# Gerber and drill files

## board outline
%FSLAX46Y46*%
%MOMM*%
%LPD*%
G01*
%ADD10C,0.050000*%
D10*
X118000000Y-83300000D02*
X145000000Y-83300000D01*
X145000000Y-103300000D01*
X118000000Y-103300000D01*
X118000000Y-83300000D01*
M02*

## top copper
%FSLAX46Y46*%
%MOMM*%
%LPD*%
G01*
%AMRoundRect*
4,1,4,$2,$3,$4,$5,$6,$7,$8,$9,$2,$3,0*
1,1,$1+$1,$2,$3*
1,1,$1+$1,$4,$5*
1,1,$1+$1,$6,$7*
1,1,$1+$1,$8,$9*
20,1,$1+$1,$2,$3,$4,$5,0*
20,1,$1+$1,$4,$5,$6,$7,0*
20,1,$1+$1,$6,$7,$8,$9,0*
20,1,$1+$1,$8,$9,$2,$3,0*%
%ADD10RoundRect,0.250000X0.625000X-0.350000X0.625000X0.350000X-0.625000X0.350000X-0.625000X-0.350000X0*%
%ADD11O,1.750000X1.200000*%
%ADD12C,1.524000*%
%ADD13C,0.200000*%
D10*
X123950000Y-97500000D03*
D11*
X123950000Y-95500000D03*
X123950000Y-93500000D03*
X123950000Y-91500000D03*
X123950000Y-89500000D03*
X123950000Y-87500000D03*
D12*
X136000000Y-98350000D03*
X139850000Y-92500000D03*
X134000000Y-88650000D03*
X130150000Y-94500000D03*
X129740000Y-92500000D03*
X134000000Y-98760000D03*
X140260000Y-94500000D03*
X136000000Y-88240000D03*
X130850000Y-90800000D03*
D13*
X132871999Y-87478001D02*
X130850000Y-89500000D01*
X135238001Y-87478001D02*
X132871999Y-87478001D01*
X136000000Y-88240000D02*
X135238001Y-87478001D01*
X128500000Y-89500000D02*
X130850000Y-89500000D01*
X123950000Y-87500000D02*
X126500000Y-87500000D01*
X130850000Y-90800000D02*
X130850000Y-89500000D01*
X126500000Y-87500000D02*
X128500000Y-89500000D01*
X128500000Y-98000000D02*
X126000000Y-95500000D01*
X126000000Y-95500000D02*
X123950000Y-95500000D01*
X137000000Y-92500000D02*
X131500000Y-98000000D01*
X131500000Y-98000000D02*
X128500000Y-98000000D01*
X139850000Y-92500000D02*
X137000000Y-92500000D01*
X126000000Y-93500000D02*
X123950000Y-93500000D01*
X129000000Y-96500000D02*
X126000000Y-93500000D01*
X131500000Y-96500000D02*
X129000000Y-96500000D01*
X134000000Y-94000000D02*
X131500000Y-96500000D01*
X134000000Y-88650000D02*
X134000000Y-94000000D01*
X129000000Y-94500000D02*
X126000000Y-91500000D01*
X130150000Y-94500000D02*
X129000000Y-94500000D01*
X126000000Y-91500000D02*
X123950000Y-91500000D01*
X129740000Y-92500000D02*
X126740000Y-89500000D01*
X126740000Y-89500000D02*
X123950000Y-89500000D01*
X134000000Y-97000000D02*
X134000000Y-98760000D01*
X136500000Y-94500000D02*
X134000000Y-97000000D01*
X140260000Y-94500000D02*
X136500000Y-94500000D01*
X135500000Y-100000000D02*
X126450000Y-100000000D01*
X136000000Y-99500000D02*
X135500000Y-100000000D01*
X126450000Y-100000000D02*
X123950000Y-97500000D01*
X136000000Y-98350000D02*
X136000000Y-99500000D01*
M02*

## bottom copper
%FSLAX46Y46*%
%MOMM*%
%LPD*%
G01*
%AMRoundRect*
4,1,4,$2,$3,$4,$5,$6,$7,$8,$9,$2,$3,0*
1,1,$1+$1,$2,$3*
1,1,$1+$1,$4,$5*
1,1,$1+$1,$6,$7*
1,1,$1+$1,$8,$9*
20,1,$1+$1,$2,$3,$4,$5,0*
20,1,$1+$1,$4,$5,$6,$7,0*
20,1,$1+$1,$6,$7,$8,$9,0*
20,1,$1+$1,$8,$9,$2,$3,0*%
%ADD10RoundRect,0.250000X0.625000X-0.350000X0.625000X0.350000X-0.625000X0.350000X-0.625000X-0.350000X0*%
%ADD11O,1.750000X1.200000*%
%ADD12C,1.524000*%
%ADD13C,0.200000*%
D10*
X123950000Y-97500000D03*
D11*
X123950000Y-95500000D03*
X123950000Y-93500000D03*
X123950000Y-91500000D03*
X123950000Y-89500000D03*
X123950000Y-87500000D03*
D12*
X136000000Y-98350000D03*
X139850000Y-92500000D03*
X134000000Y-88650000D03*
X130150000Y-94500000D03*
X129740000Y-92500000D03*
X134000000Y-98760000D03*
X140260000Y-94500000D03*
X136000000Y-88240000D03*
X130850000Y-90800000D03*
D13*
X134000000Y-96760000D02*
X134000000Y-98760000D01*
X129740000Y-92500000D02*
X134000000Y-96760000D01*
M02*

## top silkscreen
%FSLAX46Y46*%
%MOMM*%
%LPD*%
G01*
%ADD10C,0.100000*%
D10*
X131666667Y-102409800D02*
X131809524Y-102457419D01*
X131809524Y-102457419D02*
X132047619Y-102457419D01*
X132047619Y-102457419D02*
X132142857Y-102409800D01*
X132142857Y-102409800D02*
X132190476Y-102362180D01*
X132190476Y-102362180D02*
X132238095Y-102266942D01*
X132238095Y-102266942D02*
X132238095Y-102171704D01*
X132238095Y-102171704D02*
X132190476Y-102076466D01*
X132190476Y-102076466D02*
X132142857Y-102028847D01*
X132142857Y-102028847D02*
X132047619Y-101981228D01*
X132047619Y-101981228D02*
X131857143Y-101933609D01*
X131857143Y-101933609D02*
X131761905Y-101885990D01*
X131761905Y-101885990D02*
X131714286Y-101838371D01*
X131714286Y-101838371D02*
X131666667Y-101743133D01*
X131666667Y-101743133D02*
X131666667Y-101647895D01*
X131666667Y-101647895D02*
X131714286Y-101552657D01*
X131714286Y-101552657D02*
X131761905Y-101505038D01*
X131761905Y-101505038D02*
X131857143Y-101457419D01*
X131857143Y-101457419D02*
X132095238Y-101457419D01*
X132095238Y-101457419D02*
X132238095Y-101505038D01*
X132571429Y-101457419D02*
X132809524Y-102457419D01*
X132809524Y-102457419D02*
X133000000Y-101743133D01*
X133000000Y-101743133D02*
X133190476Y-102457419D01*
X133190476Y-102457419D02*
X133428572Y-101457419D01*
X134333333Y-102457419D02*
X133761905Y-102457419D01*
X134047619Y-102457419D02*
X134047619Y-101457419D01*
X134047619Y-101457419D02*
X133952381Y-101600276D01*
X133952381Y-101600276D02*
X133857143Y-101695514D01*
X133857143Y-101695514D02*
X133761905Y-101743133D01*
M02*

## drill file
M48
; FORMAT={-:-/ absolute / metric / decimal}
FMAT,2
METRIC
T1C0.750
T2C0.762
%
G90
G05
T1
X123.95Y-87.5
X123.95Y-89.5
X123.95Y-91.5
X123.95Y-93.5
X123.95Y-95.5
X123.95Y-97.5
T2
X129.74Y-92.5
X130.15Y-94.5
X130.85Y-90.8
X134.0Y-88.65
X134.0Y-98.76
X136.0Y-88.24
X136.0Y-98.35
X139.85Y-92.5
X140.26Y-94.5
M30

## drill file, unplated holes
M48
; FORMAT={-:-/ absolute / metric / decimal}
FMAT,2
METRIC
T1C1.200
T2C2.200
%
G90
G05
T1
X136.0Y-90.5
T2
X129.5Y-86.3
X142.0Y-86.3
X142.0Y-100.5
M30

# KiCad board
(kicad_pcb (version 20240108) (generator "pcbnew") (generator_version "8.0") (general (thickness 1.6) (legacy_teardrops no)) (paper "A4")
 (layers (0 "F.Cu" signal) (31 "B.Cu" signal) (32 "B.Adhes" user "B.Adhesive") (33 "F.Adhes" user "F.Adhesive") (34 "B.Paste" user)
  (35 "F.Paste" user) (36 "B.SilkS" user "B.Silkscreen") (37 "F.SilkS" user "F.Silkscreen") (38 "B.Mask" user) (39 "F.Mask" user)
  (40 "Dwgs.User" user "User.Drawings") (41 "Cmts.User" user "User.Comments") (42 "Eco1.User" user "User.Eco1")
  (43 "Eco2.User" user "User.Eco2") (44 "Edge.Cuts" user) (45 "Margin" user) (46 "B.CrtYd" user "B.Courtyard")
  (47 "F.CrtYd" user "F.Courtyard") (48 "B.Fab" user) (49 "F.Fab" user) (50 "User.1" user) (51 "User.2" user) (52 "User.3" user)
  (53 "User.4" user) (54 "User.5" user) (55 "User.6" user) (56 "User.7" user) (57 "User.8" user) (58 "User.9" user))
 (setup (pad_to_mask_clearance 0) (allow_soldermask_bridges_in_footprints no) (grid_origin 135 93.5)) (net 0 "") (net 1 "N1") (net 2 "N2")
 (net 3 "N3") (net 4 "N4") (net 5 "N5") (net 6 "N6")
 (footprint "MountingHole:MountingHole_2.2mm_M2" (layer "F.Cu") (at 129.5 86.3)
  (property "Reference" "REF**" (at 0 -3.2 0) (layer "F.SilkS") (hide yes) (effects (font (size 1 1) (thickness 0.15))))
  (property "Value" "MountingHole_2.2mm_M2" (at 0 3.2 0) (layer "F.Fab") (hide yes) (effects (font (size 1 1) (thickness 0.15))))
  (pad "" np_thru_hole circle (at 0 0) (size 2.2 2.2) (drill 2.2) (layers "F&B.Cu" "*.Mask")))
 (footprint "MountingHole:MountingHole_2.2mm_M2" (layer "F.Cu") (at 142 100.5)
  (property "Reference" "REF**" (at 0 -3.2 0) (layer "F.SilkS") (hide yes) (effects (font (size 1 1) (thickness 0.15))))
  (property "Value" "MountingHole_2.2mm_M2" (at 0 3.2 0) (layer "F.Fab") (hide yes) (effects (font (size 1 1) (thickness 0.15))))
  (pad "" np_thru_hole circle (at 0 0) (size 2.2 2.2) (drill 2.2) (layers "F&B.Cu" "*.Mask")))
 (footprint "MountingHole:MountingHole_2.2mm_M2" (layer "F.Cu") (at 142 86.3)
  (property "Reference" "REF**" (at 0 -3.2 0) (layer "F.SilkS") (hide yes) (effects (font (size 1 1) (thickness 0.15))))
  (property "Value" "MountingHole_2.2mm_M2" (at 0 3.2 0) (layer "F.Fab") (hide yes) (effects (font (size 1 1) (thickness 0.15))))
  (pad "" np_thru_hole circle (at 0 0) (size 2.2 2.2) (drill 2.2) (layers "F&B.Cu" "*.Mask")))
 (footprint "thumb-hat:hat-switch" (layer "F.Cu") (at 135 93.5)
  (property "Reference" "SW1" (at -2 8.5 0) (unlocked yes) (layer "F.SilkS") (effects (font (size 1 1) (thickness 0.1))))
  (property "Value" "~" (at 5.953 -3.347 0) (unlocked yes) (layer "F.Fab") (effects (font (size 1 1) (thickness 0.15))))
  (pad "" np_thru_hole circle (at 1 -3) (size 1.2 1.2) (drill 1.2) (layers "*.Mask"))
  (pad "1" thru_hole circle (at 1 4.85) (size 1.524 1.524) (drill 0.762) (layers "*.Cu" "*.Mask") (remove_unused_layers no) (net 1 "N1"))
  (pad "2" thru_hole circle (at 4.85 -1) (size 1.524 1.524) (drill 0.762) (layers "*.Cu" "*.Mask") (remove_unused_layers no) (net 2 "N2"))
  (pad "3" thru_hole circle (at -1 -4.85) (size 1.524 1.524) (drill 0.762) (layers "*.Cu" "*.Mask") (remove_unused_layers no) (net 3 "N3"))
  (pad "4" thru_hole circle (at -4.85 1) (size 1.524 1.524) (drill 0.762) (layers "*.Cu" "*.Mask") (remove_unused_layers no) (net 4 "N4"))
  (pad "5" thru_hole circle (at -5.26 -1) (size 1.524 1.524) (drill 0.762) (layers "*.Cu" "*.Mask") (remove_unused_layers no) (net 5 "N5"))
  (pad "5" thru_hole circle (at -1 5.26) (size 1.524 1.524) (drill 0.762) (layers "*.Cu" "*.Mask") (remove_unused_layers no) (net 5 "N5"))
  (pad "5" thru_hole circle (at 5.26 1) (size 1.524 1.524) (drill 0.762) (layers "*.Cu" "*.Mask") (remove_unused_layers no) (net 5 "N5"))
  (pad "6" thru_hole circle (at 1 -5.26) (size 1.524 1.524) (drill 0.762) (layers "*.Cu" "*.Mask") (remove_unused_layers no) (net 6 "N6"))
  (pad "7" thru_hole circle (at -4.15 -2.7) (size 1.524 1.524) (drill 0.762) (layers "*.Cu" "*.Mask") (remove_unused_layers no) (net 6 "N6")))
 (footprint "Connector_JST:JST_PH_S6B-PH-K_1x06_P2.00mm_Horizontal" (layer "B.Cu") (at 123.95 97.5 90)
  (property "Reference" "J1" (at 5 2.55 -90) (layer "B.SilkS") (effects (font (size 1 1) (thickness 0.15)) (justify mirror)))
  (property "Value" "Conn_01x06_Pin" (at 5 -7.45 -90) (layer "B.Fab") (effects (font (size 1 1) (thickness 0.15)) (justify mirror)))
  (pad "1" thru_hole roundrect (at 0 0 90) (size 1.2 1.75) (drill 0.75) (layers "*.Cu" "*.Mask") (remove_unused_layers no)
   (roundrect_rratio 0.208333) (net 1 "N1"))
  (pad "2" thru_hole oval (at 2 0 90) (size 1.2 1.75) (drill 0.75) (layers "*.Cu" "*.Mask") (remove_unused_layers no) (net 2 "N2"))
  (pad "3" thru_hole oval (at 4 0 90) (size 1.2 1.75) (drill 0.75) (layers "*.Cu" "*.Mask") (remove_unused_layers no) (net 3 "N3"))
  (pad "4" thru_hole oval (at 6 0 90) (size 1.2 1.75) (drill 0.75) (layers "*.Cu" "*.Mask") (remove_unused_layers no) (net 4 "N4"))
  (pad "5" thru_hole oval (at 8 0 90) (size 1.2 1.75) (drill 0.75) (layers "*.Cu" "*.Mask") (remove_unused_layers no) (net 5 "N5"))
  (pad "6" thru_hole oval (at 10 0 90) (size 1.2 1.75) (drill 0.75) (layers "*.Cu" "*.Mask") (remove_unused_layers no) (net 6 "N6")))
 (gr_rect (start 118 83.3) (end 145 103.3) (stroke (width 0.05) (type default)) (fill none) (layer "Edge.Cuts"))
 (segment (start 132.871999 87.478001) (end 130.85 89.5) (width 0.2) (layer "F.Cu") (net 6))
 (segment (start 130.85 90.8) (end 130.85 89.5) (width 0.2) (layer "F.Cu") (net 6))
 (segment (start 136 88.24) (end 135.238001 87.478001) (width 0.2) (layer "F.Cu") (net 6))
 (segment (start 135.238001 87.478001) (end 132.871999 87.478001) (width 0.2) (layer "F.Cu") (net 6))
 (segment (start 123.95 87.5) (end 126.5 87.5) (width 0.2) (layer "F.Cu") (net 6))
 (segment (start 128.5 89.5) (end 130.85 89.5) (width 0.2) (layer "F.Cu") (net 6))
 (segment (start 126.5 87.5) (end 128.5 89.5) (width 0.2) (layer "F.Cu") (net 6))
 (segment (start 136 99.5) (end 135.5 100) (width 0.2) (layer "F.Cu") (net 1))
 (segment (start 136 98.35) (end 136 99.5) (width 0.2) (layer "F.Cu") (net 1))
 (segment (start 135.5 100) (end 126.45 100) (width 0.2) (layer "F.Cu") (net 1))
 (segment (start 126.45 100) (end 123.95 97.5) (width 0.2) (layer "F.Cu") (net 1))
 (segment (start 140.26 94.5) (end 136.5 94.5) (width 0.2) (layer "F.Cu") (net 5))
 (segment (start 129.74 92.5) (end 126.74 89.5) (width 0.2) (layer "F.Cu") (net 5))
 (segment (start 126.74 89.5) (end 123.95 89.5) (width 0.2) (layer "F.Cu") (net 5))
 (segment (start 136.5 94.5) (end 134 97) (width 0.2) (layer "F.Cu") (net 5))
 (segment (start 134 97) (end 134 98.76) (width 0.2) (layer "F.Cu") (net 5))
 (segment (start 129.74 92.5) (end 134 96.76) (width 0.2) (layer "B.Cu") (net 5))
 (segment (start 134 96.76) (end 134 98.76) (width 0.2) (layer "B.Cu") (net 5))
 (segment (start 134 94) (end 131.5 96.5) (width 0.2) (layer "F.Cu") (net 3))
 (segment (start 129 96.5) (end 126 93.5) (width 0.2) (layer "F.Cu") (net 3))
 (segment (start 134 88.65) (end 134 94) (width 0.2) (layer "F.Cu") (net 3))
 (segment (start 126 93.5) (end 123.95 93.5) (width 0.2) (layer "F.Cu") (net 3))
 (segment (start 131.5 96.5) (end 129 96.5) (width 0.2) (layer "F.Cu") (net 3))
 (segment (start 128.5 98) (end 126 95.5) (width 0.2) (layer "F.Cu") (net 2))
 (segment (start 131.5 98) (end 128.5 98) (width 0.2) (layer "F.Cu") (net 2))
 (segment (start 139.85 92.5) (end 137 92.5) (width 0.2) (layer "F.Cu") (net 2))
 (segment (start 126 95.5) (end 123.95 95.5) (width 0.2) (layer "F.Cu") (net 2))
 (segment (start 137 92.5) (end 131.5 98) (width 0.2) (layer "F.Cu") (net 2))
 (segment (start 130.15 94.5) (end 129 94.5) (width 0.2) (layer "F.Cu") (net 4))
 (segment (start 129 94.5) (end 126 91.5) (width 0.2) (layer "F.Cu") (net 4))
 (segment (start 126 91.5) (end 123.95 91.5) (width 0.2) (layer "F.Cu") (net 4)))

